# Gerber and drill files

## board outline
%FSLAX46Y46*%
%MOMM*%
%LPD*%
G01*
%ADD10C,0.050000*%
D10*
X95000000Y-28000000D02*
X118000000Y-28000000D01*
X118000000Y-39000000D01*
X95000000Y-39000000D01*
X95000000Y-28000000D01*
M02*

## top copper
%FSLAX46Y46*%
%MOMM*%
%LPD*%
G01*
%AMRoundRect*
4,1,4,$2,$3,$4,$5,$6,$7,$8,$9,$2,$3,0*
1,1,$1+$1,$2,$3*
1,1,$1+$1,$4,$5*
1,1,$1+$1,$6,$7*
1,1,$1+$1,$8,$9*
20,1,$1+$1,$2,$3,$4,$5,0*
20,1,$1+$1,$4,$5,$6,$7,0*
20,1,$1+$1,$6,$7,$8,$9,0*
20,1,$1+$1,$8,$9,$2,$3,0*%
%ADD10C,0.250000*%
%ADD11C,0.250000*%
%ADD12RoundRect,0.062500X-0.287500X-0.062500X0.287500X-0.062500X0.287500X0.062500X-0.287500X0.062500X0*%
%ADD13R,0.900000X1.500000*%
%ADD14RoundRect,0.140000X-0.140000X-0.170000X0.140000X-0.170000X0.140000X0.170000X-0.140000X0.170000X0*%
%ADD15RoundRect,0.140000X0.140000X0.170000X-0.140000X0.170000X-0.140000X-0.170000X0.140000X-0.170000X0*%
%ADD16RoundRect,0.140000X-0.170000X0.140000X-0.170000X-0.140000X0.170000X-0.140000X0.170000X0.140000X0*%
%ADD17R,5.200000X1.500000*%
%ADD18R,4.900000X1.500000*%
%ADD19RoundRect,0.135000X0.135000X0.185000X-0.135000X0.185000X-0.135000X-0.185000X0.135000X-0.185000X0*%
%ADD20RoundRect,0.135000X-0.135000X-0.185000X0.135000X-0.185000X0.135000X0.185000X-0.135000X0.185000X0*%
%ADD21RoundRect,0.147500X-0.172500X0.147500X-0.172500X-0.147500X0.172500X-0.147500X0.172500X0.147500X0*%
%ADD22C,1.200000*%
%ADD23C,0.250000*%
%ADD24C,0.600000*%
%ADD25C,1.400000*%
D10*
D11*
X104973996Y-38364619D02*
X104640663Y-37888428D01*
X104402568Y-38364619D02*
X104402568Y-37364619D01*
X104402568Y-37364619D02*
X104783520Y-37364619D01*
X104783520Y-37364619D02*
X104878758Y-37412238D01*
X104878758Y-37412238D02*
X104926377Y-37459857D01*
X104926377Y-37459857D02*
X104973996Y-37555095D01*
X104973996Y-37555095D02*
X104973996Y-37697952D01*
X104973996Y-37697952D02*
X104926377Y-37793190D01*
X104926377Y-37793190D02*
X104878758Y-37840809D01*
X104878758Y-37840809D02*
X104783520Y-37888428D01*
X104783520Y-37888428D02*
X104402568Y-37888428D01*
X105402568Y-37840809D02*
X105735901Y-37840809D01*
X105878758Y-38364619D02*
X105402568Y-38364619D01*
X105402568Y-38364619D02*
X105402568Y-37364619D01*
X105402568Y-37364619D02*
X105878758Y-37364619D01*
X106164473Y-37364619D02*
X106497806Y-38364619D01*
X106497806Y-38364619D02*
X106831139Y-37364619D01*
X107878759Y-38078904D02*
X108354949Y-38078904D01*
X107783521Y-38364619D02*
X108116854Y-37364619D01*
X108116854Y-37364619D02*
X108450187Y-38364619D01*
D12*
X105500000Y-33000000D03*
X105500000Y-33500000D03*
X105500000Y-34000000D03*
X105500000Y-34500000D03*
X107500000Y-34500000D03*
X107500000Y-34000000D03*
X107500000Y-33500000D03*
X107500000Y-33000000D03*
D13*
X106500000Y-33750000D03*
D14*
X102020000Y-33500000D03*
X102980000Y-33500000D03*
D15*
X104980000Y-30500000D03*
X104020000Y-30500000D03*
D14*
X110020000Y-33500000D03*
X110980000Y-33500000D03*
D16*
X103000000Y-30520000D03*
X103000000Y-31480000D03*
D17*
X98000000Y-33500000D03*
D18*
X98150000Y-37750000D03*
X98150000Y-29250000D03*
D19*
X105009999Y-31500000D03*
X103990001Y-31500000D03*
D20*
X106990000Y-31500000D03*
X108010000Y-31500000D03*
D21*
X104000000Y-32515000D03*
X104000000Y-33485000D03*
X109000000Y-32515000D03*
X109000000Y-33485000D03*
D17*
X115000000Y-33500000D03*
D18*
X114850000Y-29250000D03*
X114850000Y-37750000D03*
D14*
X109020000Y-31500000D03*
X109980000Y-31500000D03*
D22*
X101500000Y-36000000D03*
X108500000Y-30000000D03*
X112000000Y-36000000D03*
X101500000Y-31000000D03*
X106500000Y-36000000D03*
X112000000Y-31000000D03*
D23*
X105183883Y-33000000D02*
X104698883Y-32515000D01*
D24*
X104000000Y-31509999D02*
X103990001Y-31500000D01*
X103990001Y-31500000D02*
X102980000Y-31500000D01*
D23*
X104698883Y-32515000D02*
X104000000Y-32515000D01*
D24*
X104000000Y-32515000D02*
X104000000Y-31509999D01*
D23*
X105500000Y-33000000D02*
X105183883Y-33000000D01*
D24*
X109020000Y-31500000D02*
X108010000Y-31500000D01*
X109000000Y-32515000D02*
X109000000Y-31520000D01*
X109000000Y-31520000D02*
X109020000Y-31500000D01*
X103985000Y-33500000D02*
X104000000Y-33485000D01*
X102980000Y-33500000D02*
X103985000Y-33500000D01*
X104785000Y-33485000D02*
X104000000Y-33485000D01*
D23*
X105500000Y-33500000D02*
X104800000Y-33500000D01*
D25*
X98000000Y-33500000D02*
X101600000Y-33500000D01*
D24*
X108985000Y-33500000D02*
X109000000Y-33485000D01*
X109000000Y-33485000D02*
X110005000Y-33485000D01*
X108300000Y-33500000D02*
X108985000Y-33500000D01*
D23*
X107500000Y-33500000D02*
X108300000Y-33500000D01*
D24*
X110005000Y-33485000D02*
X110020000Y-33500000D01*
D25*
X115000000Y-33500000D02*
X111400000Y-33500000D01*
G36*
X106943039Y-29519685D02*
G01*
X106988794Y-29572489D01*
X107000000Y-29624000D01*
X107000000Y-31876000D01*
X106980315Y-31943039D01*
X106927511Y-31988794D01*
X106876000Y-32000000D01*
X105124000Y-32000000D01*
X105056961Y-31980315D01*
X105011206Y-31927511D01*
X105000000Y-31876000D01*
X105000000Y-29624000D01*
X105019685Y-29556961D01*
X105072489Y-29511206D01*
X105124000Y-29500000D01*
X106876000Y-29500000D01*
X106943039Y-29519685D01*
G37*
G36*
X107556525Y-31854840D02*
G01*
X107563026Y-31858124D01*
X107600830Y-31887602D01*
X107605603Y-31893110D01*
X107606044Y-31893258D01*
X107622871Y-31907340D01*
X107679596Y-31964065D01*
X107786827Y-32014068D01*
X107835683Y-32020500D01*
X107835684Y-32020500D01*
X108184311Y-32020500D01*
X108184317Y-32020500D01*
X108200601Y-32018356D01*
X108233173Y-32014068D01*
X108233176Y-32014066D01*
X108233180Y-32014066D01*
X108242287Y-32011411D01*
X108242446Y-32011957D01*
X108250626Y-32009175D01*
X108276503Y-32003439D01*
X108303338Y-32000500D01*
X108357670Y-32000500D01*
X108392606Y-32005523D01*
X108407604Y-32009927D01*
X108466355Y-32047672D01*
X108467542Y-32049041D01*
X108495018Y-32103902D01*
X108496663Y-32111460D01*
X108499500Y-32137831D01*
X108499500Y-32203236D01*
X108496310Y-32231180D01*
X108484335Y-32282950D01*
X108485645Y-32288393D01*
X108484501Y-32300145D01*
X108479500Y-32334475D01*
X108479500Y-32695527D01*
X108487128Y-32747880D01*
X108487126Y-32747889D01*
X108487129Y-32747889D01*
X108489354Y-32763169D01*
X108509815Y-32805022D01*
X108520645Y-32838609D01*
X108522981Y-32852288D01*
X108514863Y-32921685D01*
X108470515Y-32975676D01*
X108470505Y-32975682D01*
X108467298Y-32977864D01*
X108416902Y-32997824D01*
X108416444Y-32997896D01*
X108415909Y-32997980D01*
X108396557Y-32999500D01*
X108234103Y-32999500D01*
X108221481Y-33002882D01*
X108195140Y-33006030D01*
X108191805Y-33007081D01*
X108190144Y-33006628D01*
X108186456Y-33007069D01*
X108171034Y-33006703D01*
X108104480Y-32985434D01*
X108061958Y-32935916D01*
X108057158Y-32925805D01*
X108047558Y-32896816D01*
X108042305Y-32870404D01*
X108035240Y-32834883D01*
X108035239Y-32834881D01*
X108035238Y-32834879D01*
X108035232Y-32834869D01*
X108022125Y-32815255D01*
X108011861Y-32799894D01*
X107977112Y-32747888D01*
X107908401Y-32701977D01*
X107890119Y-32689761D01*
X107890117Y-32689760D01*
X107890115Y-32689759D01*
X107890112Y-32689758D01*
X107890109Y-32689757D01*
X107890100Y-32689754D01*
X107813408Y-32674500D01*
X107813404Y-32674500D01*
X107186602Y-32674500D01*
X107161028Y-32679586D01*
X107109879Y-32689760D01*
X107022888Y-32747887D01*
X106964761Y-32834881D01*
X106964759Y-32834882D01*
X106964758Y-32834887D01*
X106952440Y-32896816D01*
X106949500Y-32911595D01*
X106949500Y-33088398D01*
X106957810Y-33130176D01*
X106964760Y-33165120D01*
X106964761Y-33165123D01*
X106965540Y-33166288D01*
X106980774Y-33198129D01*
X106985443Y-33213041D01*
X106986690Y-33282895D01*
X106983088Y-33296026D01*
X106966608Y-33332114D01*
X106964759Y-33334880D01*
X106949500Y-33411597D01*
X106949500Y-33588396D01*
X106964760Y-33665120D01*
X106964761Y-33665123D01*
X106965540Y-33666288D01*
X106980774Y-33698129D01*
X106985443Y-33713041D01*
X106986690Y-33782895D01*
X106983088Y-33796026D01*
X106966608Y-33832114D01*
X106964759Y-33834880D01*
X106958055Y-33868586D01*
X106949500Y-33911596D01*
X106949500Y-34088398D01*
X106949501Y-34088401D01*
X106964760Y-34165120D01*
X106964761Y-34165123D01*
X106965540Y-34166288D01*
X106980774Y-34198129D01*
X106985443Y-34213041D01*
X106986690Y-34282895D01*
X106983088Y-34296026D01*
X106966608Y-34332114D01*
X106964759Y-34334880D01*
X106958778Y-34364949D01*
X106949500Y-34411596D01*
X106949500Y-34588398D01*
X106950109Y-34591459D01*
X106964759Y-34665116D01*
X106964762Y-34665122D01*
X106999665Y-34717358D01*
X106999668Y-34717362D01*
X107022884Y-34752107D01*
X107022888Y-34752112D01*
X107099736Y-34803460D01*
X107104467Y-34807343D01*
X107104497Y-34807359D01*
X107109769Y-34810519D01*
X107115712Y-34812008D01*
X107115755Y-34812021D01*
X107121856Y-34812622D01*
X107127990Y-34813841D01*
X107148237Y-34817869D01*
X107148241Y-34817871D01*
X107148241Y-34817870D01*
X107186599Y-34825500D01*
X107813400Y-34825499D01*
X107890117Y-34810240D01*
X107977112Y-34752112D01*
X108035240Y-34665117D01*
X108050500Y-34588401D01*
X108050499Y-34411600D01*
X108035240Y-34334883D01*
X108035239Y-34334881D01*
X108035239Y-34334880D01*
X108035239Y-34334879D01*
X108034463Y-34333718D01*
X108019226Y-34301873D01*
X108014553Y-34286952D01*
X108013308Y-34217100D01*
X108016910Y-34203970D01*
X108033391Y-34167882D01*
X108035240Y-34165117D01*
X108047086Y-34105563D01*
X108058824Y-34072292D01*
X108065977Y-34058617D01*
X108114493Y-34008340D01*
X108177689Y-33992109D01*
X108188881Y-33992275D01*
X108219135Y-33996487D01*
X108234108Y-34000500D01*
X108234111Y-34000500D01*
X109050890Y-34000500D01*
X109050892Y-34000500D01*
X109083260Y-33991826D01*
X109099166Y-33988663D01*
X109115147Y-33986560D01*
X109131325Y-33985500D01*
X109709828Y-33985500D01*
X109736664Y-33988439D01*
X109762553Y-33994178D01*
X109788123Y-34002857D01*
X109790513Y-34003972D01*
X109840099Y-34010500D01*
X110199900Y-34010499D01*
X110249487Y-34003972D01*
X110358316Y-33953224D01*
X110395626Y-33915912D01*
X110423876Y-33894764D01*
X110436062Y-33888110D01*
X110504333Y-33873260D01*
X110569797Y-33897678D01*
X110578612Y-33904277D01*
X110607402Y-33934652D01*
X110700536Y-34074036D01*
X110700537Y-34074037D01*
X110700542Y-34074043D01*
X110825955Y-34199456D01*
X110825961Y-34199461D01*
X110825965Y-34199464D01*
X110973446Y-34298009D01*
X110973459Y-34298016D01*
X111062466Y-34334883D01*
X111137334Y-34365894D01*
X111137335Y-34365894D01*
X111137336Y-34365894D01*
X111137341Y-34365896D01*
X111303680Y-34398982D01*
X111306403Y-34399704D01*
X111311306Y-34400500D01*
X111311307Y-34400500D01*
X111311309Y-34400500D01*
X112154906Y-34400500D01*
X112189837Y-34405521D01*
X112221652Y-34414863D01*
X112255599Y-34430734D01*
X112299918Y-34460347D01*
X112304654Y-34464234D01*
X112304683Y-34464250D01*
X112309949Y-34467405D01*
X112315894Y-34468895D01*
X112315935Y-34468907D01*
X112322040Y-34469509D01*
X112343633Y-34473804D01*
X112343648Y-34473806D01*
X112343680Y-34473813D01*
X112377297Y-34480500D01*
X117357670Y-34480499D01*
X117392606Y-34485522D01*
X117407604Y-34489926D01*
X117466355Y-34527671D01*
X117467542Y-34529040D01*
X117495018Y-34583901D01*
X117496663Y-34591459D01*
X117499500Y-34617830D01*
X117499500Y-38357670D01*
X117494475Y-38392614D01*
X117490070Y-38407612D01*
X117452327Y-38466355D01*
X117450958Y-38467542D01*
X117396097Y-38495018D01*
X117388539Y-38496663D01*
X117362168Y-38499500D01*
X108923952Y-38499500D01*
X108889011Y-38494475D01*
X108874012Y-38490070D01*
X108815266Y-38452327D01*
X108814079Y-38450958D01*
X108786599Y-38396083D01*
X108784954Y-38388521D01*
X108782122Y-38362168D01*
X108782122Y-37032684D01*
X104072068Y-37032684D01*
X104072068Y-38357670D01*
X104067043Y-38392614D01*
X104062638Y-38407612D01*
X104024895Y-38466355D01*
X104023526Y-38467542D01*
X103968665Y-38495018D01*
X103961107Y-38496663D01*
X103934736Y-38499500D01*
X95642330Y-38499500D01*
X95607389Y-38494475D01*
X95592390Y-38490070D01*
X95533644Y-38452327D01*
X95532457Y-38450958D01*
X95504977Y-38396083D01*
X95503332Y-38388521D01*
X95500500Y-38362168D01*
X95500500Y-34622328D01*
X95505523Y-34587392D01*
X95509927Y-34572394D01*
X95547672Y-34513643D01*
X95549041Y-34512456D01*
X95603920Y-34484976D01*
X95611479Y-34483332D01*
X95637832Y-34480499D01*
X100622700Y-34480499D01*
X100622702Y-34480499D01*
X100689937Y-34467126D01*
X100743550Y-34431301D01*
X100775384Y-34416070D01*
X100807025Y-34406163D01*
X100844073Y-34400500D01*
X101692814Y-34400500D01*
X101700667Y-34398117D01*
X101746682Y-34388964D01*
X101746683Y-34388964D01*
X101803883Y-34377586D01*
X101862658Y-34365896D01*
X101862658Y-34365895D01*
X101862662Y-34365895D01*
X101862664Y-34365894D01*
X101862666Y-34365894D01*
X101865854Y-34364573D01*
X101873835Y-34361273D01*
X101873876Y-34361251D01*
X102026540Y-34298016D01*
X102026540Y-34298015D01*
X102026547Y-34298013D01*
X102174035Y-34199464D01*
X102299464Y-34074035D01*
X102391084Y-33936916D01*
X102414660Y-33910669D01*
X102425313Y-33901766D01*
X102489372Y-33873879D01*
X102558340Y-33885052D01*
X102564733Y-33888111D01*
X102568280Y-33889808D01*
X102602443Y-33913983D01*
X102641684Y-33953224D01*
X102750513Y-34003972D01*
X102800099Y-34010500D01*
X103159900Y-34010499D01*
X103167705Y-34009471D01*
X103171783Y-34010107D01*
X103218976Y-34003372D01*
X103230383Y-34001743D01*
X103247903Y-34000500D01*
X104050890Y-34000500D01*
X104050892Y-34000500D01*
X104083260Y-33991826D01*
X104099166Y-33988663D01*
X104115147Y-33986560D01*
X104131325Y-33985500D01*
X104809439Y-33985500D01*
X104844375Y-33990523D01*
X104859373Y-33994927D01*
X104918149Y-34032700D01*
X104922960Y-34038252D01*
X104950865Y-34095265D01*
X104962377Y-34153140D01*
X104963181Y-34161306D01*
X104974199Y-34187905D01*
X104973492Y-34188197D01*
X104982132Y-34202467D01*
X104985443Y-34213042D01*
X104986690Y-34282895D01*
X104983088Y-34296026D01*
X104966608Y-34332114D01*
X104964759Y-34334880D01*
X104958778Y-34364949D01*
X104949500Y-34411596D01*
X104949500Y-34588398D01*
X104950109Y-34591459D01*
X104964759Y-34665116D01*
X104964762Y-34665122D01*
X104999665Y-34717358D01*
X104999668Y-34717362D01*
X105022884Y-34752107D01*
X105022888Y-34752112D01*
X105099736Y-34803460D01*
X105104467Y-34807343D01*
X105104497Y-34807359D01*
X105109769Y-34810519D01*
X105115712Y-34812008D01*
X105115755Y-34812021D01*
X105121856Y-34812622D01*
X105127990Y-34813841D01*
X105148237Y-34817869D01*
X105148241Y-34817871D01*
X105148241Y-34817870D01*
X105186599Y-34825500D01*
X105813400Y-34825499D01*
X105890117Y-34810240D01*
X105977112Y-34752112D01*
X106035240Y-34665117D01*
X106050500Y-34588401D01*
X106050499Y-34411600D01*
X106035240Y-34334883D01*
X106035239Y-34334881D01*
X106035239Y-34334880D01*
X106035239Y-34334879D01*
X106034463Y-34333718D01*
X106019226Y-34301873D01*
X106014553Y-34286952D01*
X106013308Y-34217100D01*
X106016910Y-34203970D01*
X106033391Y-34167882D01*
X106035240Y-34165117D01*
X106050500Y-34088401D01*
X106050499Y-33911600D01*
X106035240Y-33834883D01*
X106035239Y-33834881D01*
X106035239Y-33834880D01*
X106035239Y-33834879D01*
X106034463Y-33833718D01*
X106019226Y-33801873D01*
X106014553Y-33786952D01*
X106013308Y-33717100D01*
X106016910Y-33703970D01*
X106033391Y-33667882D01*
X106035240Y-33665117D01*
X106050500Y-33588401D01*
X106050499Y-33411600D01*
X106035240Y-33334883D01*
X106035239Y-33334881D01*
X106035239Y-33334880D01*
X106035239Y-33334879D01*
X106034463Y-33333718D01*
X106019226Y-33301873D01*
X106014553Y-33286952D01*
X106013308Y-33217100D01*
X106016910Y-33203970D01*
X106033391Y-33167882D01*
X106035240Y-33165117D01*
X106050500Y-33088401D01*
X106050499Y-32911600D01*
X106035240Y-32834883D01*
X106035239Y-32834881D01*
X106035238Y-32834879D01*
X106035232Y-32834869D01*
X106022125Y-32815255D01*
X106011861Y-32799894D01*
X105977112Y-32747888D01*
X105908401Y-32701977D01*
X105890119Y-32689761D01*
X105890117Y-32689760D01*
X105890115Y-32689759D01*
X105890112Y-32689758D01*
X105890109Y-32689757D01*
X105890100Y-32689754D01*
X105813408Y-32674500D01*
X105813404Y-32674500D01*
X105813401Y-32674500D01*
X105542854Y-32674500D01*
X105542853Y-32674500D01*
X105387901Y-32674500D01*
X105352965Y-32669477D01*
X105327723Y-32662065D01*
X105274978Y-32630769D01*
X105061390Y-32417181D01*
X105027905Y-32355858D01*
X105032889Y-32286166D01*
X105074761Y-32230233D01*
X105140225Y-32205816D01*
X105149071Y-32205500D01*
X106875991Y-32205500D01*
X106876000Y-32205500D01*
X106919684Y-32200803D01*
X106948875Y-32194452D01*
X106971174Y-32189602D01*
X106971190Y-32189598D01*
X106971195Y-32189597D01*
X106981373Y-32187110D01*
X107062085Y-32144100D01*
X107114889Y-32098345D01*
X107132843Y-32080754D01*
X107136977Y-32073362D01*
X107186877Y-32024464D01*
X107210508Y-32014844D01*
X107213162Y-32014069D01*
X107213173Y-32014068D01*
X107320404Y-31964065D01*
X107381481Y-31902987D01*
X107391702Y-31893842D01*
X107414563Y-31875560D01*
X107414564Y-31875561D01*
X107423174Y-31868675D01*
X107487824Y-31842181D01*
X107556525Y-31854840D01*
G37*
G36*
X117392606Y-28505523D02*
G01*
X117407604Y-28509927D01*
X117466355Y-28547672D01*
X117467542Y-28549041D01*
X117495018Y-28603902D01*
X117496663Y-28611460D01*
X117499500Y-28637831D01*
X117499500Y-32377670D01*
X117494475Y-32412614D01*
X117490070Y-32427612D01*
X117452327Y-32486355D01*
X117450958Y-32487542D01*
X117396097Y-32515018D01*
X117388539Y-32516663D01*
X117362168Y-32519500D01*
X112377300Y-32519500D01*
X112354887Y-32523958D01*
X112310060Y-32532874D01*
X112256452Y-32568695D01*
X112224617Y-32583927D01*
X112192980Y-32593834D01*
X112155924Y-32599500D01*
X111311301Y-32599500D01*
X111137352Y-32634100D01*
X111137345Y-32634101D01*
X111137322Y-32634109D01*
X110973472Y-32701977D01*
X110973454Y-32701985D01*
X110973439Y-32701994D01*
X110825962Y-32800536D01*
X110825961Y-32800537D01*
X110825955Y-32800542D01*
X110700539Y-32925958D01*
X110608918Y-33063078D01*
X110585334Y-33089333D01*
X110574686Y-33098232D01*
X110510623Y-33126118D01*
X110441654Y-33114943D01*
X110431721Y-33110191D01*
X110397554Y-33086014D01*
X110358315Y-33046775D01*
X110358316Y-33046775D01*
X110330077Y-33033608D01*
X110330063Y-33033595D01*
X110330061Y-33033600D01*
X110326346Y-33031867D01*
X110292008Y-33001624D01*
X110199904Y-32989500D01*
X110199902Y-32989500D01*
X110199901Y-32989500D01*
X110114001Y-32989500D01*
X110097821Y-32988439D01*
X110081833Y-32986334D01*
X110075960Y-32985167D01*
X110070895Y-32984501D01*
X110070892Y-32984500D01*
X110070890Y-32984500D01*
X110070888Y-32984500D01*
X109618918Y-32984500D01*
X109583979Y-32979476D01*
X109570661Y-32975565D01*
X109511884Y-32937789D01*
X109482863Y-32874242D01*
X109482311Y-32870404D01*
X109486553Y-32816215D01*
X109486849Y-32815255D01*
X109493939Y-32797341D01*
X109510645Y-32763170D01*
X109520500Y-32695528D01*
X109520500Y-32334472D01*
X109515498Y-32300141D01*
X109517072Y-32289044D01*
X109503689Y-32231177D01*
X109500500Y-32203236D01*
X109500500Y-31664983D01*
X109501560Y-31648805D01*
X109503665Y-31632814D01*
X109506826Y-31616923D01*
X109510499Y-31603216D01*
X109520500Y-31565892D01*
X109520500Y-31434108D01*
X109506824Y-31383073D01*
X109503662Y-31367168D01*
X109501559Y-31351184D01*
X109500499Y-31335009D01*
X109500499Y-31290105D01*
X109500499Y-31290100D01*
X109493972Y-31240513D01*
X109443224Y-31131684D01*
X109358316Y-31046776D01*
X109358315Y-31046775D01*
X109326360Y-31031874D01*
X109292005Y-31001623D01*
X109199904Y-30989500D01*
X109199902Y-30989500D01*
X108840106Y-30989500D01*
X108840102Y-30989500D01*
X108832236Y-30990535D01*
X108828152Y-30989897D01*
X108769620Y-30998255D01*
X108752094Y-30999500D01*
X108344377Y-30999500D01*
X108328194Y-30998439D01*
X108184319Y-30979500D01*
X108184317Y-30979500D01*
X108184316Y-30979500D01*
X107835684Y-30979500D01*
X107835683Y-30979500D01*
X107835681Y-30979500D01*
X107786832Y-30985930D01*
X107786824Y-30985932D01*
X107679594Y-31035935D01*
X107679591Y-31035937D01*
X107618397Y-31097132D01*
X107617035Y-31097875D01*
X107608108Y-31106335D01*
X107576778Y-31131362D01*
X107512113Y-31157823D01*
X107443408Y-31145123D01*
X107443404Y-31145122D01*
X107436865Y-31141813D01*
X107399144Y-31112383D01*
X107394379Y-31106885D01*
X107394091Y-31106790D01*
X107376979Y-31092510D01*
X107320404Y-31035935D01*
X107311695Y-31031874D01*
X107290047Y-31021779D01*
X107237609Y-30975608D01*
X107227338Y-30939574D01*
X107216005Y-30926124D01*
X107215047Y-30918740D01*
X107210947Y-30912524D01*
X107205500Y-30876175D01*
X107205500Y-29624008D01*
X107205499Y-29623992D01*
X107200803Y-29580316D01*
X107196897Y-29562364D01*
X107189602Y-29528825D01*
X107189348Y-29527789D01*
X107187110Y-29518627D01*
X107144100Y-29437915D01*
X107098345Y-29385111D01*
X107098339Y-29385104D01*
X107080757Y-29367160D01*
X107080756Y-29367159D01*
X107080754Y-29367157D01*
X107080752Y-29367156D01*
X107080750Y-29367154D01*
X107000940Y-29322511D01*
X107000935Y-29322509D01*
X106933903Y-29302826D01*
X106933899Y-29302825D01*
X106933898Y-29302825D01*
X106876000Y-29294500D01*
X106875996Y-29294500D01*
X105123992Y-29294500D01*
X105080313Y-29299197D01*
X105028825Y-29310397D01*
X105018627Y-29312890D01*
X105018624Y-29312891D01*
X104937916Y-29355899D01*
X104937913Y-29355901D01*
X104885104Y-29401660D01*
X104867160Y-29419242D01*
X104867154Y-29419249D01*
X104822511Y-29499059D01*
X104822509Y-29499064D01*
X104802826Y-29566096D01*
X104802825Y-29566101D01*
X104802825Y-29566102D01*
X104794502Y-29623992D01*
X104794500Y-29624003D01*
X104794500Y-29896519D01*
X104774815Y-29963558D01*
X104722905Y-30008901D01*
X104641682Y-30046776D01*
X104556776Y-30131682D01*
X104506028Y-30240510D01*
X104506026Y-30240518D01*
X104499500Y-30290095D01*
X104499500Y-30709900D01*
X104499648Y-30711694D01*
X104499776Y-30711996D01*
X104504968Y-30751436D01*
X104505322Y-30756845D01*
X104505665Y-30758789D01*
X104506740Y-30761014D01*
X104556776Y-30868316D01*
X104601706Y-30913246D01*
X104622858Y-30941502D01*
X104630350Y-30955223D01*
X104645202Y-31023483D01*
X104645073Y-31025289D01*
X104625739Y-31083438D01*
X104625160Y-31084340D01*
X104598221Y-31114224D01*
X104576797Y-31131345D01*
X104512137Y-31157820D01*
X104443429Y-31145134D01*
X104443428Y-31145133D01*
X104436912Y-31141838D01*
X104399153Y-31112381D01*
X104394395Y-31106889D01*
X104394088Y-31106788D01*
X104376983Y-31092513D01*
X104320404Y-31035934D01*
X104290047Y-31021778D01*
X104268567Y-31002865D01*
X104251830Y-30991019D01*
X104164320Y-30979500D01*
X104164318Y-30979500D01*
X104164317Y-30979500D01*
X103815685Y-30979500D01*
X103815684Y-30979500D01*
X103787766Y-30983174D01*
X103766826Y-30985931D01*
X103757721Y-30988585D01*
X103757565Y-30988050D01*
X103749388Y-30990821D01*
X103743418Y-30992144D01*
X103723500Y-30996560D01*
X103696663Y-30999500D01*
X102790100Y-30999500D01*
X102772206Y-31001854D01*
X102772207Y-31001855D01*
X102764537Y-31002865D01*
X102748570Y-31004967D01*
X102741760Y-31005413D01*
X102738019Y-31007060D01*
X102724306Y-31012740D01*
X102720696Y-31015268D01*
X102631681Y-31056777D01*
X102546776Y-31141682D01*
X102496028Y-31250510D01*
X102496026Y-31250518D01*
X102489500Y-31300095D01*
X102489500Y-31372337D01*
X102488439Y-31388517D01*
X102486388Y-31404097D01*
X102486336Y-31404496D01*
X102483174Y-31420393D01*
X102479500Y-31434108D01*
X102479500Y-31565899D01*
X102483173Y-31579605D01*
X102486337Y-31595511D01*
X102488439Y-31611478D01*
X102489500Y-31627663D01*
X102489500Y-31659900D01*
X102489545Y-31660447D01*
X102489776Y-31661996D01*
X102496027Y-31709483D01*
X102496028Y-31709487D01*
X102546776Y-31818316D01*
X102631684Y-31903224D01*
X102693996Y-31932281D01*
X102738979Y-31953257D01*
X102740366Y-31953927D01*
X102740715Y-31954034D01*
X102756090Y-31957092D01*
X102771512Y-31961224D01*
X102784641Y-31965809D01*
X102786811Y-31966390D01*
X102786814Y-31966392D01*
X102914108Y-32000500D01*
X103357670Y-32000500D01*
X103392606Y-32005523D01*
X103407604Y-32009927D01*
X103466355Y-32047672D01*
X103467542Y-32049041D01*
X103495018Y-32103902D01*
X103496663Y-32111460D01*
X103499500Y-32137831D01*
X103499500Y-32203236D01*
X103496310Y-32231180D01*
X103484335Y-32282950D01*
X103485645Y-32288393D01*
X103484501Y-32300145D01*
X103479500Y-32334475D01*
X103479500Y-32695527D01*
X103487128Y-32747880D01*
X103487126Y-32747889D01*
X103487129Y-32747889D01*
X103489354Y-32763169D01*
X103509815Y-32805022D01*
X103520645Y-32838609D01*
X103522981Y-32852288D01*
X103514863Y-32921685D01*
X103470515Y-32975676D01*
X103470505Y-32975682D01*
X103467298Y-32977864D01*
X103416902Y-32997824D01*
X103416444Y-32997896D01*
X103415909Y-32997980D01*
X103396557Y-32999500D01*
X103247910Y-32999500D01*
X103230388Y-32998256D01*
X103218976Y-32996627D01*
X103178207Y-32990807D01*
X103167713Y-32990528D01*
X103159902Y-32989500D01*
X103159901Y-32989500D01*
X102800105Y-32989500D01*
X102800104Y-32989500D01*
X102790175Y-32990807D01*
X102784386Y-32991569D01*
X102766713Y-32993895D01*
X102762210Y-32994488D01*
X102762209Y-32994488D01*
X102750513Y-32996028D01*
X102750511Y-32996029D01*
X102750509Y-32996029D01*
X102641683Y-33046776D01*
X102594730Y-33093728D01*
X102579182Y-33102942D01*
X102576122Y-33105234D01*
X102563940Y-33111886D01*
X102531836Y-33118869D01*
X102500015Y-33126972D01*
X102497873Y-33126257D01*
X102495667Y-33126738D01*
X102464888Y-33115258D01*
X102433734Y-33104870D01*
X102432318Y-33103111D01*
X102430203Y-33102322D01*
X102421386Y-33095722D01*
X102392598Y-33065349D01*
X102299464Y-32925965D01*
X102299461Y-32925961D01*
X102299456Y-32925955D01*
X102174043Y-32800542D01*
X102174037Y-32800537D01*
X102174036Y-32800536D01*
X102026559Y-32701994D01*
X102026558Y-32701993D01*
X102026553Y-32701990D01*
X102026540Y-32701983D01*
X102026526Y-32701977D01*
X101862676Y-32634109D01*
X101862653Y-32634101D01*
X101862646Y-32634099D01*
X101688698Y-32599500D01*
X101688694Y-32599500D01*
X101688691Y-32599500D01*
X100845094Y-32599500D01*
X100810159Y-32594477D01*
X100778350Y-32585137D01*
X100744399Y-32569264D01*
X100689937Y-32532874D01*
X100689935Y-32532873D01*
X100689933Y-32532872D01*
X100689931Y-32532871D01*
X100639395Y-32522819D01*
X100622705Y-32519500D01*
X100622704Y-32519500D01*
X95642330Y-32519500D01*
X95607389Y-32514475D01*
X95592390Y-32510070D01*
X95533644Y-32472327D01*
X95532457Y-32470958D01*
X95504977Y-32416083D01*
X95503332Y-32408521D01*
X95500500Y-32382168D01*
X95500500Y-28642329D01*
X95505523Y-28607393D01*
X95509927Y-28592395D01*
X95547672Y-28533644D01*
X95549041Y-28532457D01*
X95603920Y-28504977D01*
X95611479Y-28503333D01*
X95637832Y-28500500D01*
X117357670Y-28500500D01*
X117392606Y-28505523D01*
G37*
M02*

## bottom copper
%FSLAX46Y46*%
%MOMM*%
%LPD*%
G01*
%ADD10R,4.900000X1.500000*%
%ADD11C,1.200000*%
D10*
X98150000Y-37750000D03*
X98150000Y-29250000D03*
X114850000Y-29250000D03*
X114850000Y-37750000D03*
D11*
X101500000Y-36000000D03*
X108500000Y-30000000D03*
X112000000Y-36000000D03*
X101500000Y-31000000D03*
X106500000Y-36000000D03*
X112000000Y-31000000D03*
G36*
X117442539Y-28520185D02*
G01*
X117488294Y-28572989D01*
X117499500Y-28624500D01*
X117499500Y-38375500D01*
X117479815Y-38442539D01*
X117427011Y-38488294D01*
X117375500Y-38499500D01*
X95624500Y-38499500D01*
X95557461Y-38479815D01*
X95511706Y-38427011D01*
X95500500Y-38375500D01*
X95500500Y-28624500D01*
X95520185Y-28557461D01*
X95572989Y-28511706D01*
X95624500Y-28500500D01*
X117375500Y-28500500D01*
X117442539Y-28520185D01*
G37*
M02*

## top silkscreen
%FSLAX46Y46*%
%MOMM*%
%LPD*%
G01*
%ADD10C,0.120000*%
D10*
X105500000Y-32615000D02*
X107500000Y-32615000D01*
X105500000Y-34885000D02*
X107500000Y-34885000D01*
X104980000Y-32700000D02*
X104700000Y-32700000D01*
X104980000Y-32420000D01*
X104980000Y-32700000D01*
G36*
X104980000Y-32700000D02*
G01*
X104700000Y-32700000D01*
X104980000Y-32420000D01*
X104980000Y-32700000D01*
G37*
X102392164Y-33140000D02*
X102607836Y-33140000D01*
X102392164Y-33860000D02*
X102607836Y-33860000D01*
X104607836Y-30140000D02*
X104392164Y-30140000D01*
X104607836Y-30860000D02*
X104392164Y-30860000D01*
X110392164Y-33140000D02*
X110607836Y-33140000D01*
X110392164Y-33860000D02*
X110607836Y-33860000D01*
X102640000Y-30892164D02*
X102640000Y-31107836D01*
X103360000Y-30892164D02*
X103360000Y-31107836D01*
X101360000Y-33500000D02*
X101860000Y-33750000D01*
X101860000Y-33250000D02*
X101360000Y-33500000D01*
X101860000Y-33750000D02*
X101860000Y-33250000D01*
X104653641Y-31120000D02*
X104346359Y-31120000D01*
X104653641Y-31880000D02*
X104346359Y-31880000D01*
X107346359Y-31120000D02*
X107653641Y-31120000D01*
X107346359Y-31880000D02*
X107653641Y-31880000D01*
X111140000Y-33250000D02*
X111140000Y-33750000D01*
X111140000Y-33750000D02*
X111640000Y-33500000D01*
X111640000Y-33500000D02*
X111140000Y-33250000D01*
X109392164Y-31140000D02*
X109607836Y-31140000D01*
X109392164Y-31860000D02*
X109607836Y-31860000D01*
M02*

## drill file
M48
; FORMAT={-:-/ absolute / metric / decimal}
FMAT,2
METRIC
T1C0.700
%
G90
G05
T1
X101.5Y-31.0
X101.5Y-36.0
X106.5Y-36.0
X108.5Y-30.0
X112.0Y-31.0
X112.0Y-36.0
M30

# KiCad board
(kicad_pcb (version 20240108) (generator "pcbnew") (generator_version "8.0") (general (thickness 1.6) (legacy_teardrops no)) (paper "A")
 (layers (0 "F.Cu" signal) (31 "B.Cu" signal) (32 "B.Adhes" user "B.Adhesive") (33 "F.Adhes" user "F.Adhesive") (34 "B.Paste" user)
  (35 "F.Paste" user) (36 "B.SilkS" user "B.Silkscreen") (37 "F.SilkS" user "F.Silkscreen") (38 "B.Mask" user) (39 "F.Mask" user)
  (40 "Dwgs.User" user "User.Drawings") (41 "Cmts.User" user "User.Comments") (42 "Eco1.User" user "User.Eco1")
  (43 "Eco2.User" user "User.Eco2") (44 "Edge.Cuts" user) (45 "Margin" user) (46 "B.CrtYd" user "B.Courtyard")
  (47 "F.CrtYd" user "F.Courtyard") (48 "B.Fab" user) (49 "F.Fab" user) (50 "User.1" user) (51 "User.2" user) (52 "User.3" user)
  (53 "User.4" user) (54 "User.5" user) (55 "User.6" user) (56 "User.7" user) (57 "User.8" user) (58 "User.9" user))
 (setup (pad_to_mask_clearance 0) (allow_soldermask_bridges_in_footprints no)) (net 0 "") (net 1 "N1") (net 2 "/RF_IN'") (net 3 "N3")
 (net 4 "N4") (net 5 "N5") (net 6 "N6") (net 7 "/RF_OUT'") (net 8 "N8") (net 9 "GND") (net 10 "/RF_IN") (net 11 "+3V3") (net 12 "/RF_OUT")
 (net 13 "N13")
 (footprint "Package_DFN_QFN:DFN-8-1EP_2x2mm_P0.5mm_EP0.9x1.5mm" (layer "F.Cu") (at 106.5 33.75)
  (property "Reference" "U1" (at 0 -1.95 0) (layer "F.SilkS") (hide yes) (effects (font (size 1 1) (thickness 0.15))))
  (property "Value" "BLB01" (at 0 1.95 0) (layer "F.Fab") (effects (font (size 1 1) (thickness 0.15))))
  (fp_line (start -1 -1.135) (end 1 -1.135) (stroke (width 0.12) (type solid)) (layer "F.SilkS"))
  (fp_line (start -1 1.135) (end 1 1.135) (stroke (width 0.12) (type solid)) (layer "F.SilkS"))
  (fp_poly
   (pts (xy -1.52 -1.05) (xy -1.8 -1.05) (xy -1.52 -1.33) (xy -1.52 -1.05)) (stroke (width 0.12) (type solid)) (fill solid)
   (layer "F.SilkS"))
  (pad "" smd roundrect (at -0.225 -0.375) (size 0.36 0.6) (layers "F.Paste") (roundrect_rratio 0.25))
  (pad "" smd roundrect (at -0.225 0.375) (size 0.36 0.6) (layers "F.Paste") (roundrect_rratio 0.25))
  (pad "" smd roundrect (at 0.225 -0.375) (size 0.36 0.6) (layers "F.Paste") (roundrect_rratio 0.25))
  (pad "" smd roundrect (at 0.225 0.375) (size 0.36 0.6) (layers "F.Paste") (roundrect_rratio 0.25))
  (pad "1" smd roundrect (at -1 -0.75) (size 0.7 0.25) (layers "F.Cu" "F.Paste" "F.Mask") (roundrect_rratio 0.25) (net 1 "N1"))
  (pad "2" smd roundrect (at -1 -0.25) (size 0.7 0.25) (layers "F.Cu" "F.Paste" "F.Mask") (roundrect_rratio 0.25) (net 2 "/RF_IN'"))
  (pad "3" smd roundrect (at -1 0.25) (size 0.7 0.25) (layers "F.Cu" "F.Paste" "F.Mask") (roundrect_rratio 0.25) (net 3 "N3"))
  (pad "4" smd roundrect (at -1 0.75) (size 0.7 0.25) (layers "F.Cu" "F.Paste" "F.Mask") (roundrect_rratio 0.25) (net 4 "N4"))
  (pad "5" smd roundrect (at 1 0.75) (size 0.7 0.25) (layers "F.Cu" "F.Paste" "F.Mask") (roundrect_rratio 0.25) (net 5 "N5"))
  (pad "6" smd roundrect (at 1 0.25) (size 0.7 0.25) (layers "F.Cu" "F.Paste" "F.Mask") (roundrect_rratio 0.25) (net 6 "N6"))
  (pad "7" smd roundrect (at 1 -0.25) (size 0.7 0.25) (layers "F.Cu" "F.Paste" "F.Mask") (roundrect_rratio 0.25) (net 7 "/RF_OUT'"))
  (pad "8" smd roundrect (at 1 -0.75) (size 0.7 0.25) (layers "F.Cu" "F.Paste" "F.Mask") (roundrect_rratio 0.25) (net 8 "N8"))
  (pad "9" smd rect (at 0 0) (size 0.9 1.5) (layers "F.Cu" "F.Mask") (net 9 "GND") (zone_connect 2)))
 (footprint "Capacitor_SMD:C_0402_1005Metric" (layer "F.Cu") (at 102.5 33.5)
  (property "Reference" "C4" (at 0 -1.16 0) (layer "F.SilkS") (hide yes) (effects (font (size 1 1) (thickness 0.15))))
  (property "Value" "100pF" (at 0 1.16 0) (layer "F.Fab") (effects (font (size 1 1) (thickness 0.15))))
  (fp_line (start -0.107836 -0.36) (end 0.107836 -0.36) (stroke (width 0.12) (type solid)) (layer "F.SilkS"))
  (fp_line (start -0.107836 0.36) (end 0.107836 0.36) (stroke (width 0.12) (type solid)) (layer "F.SilkS"))
  (pad "1" smd roundrect (at -0.48 0) (size 0.56 0.62) (layers "F.Cu" "F.Paste" "F.Mask") (roundrect_rratio 0.25) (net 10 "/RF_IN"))
  (pad "2" smd roundrect (at 0.48 0) (size 0.56 0.62) (layers "F.Cu" "F.Paste" "F.Mask") (roundrect_rratio 0.25) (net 2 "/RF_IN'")))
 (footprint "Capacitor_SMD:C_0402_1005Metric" (layer "F.Cu") (at 104.5 30.5 180)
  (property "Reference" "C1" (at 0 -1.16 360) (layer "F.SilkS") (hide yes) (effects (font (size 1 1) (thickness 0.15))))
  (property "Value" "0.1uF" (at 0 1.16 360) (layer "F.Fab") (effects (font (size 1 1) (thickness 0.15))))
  (fp_line (start -0.107836 0.36) (end 0.107836 0.36) (stroke (width 0.12) (type solid)) (layer "F.SilkS"))
  (fp_line (start -0.107836 -0.36) (end 0.107836 -0.36) (stroke (width 0.12) (type solid)) (layer "F.SilkS"))
  (pad "1" smd roundrect (at -0.48 0 180) (size 0.56 0.62) (layers "F.Cu" "F.Paste" "F.Mask") (roundrect_rratio 0.25) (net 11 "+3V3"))
  (pad "2" smd roundrect (at 0.48 0 180) (size 0.56 0.62) (layers "F.Cu" "F.Paste" "F.Mask") (roundrect_rratio 0.25) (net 9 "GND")))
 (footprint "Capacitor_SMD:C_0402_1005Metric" (layer "F.Cu") (at 110.5 33.5)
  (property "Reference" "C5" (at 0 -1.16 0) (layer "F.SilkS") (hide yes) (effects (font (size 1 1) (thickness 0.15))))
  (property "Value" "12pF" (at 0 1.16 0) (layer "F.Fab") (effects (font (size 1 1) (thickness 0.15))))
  (fp_line (start -0.107836 -0.36) (end 0.107836 -0.36) (stroke (width 0.12) (type solid)) (layer "F.SilkS"))
  (fp_line (start -0.107836 0.36) (end 0.107836 0.36) (stroke (width 0.12) (type solid)) (layer "F.SilkS"))
  (pad "1" smd roundrect (at -0.48 0) (size 0.56 0.62) (layers "F.Cu" "F.Paste" "F.Mask") (roundrect_rratio 0.25) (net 7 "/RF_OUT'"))
  (pad "2" smd roundrect (at 0.48 0) (size 0.56 0.62) (layers "F.Cu" "F.Paste" "F.Mask") (roundrect_rratio 0.25) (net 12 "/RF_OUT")))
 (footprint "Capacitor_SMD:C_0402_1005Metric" (layer "F.Cu") (at 103 31 -90)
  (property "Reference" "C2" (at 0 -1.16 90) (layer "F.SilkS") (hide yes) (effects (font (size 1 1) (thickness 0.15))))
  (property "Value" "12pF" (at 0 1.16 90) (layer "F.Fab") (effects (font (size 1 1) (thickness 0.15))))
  (fp_line (start -0.107836 0.36) (end 0.107836 0.36) (stroke (width 0.12) (type solid)) (layer "F.SilkS"))
  (fp_line (start -0.107836 -0.36) (end 0.107836 -0.36) (stroke (width 0.12) (type solid)) (layer "F.SilkS"))
  (pad "1" smd roundrect (at -0.48 0 270) (size 0.56 0.62) (layers "F.Cu" "F.Paste" "F.Mask") (roundrect_rratio 0.25) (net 9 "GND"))
  (pad "2" smd roundrect (at 0.48 0 270) (size 0.56 0.62) (layers "F.Cu" "F.Paste" "F.Mask") (roundrect_rratio 0.25) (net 1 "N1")))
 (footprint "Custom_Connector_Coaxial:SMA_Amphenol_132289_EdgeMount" (layer "F.Cu") (at 98.15 33.5 180)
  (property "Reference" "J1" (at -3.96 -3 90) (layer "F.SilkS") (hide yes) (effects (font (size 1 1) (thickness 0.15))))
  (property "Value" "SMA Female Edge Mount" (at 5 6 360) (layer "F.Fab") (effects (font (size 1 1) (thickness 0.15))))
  (fp_line (start -3.21 0) (end -3.71 -0.25) (stroke (width 0.12) (type solid)) (layer "F.SilkS"))
  (fp_line (start -3.71 0.25) (end -3.21 0) (stroke (width 0.12) (type solid)) (layer "F.SilkS"))
  (fp_line (start -3.71 -0.25) (end -3.71 0.25) (stroke (width 0.12) (type solid)) (layer "F.SilkS"))
  (pad "1" smd rect (at 0.15 0 270) (size 1.5 5.2) (layers "F.Cu" "F.Paste" "F.Mask") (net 10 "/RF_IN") (clearance 0.23))
  (pad "2" smd rect (at 0 -4.25 270) (size 1.5 4.9) (layers "F.Cu" "F.Paste" "F.Mask") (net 9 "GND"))
  (pad "2" smd rect (at 0 -4.25 270) (size 1.5 4.9) (layers "B.Cu" "B.Paste" "B.Mask") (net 9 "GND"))
  (pad "2" smd rect (at 0 4.25 270) (size 1.5 4.9) (layers "F.Cu" "F.Paste" "F.Mask") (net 9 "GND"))
  (pad "2" smd rect (at 0 4.25 270) (size 1.5 4.9) (layers "B.Cu" "B.Paste" "B.Mask") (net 9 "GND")))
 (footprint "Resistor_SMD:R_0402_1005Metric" (layer "F.Cu") (at 104.5 31.5 180)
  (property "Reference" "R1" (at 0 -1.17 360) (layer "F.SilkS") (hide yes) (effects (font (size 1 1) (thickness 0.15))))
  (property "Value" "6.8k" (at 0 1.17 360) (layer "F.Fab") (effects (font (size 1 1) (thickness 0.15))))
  (fp_line (start -0.153641 0.38) (end 0.153641 0.38) (stroke (width 0.12) (type solid)) (layer "F.SilkS"))
  (fp_line (start -0.153641 -0.38) (end 0.153641 -0.38) (stroke (width 0.12) (type solid)) (layer "F.SilkS"))
  (pad "1" smd roundrect (at -0.509999 0 180) (size 0.54 0.64) (layers "F.Cu" "F.Paste" "F.Mask") (roundrect_rratio 0.25) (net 11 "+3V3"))
  (pad "2" smd roundrect (at 0.509999 0 180) (size 0.54 0.64) (layers "F.Cu" "F.Paste" "F.Mask") (roundrect_rratio 0.25) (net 1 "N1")))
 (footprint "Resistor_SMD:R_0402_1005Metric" (layer "F.Cu") (at 107.5 31.5)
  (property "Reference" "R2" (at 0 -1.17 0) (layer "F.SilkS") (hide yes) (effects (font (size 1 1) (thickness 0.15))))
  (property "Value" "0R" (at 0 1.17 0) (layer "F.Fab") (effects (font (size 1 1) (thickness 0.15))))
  (fp_line (start -0.153641 -0.38) (end 0.153641 -0.38) (stroke (width 0.12) (type solid)) (layer "F.SilkS"))
  (fp_line (start -0.153641 0.38) (end 0.153641 0.38) (stroke (width 0.12) (type solid)) (layer "F.SilkS"))
  (pad "1" smd roundrect (at -0.51 0) (size 0.54 0.64) (layers "F.Cu" "F.Paste" "F.Mask") (roundrect_rratio 0.25) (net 11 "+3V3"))
  (pad "2" smd roundrect (at 0.51 0) (size 0.54 0.64) (layers "F.Cu" "F.Paste" "F.Mask") (roundrect_rratio 0.25) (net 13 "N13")))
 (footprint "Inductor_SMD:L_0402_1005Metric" (layer "F.Cu") (at 104 33 -90)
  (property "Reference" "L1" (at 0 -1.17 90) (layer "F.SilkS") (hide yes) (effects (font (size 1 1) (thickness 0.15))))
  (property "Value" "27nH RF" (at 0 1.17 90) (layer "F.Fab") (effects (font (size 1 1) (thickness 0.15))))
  (pad "1" smd roundrect (at -0.485 0 270) (size 0.59 0.64) (layers "F.Cu" "F.Paste" "F.Mask") (roundrect_rratio 0.25) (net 1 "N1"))
  (pad "2" smd roundrect (at 0.485 0 270) (size 0.59 0.64) (layers "F.Cu" "F.Paste" "F.Mask") (roundrect_rratio 0.25) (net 2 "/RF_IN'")))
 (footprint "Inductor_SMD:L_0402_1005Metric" (layer "F.Cu") (at 109 33 -90)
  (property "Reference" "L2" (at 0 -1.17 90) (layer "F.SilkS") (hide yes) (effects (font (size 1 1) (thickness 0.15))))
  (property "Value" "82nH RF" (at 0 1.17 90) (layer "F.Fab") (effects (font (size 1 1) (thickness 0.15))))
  (pad "1" smd roundrect (at -0.485 0 270) (size 0.59 0.64) (layers "F.Cu" "F.Paste" "F.Mask") (roundrect_rratio 0.25) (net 13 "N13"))
  (pad "2" smd roundrect (at 0.485 0 270) (size 0.59 0.64) (layers "F.Cu" "F.Paste" "F.Mask") (roundrect_rratio 0.25) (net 7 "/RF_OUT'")))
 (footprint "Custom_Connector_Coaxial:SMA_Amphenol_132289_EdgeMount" (layer "F.Cu") (at 114.85 33.5)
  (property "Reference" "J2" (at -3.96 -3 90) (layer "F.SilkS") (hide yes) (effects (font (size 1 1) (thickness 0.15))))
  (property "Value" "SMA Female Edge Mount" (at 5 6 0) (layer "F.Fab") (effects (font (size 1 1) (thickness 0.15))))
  (fp_line (start -3.71 -0.25) (end -3.71 0.25) (stroke (width 0.12) (type solid)) (layer "F.SilkS"))
  (fp_line (start -3.71 0.25) (end -3.21 0) (stroke (width 0.12) (type solid)) (layer "F.SilkS"))
  (fp_line (start -3.21 0) (end -3.71 -0.25) (stroke (width 0.12) (type solid)) (layer "F.SilkS"))
  (pad "1" smd rect (at 0.15 0 90) (size 1.5 5.2) (layers "F.Cu" "F.Paste" "F.Mask") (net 12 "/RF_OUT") (clearance 0.23))
  (pad "2" smd rect (at 0 -4.25 90) (size 1.5 4.9) (layers "F.Cu" "F.Paste" "F.Mask") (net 9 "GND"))
  (pad "2" smd rect (at 0 -4.25 90) (size 1.5 4.9) (layers "B.Cu" "B.Paste" "B.Mask") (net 9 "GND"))
  (pad "2" smd rect (at 0 4.25 90) (size 1.5 4.9) (layers "F.Cu" "F.Paste" "F.Mask") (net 9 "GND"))
  (pad "2" smd rect (at 0 4.25 90) (size 1.5 4.9) (layers "B.Cu" "B.Paste" "B.Mask") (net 9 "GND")))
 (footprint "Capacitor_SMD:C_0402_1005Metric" (layer "F.Cu") (at 109.5 31.5)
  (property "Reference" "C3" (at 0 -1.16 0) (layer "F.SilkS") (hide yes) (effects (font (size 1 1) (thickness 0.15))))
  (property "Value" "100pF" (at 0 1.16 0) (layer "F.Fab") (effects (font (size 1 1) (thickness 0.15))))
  (fp_line (start -0.107836 -0.36) (end 0.107836 -0.36) (stroke (width 0.12) (type solid)) (layer "F.SilkS"))
  (fp_line (start -0.107836 0.36) (end 0.107836 0.36) (stroke (width 0.12) (type solid)) (layer "F.SilkS"))
  (pad "1" smd roundrect (at -0.48 0) (size 0.56 0.62) (layers "F.Cu" "F.Paste" "F.Mask") (roundrect_rratio 0.25) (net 13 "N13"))
  (pad "2" smd roundrect (at 0.48 0) (size 0.56 0.62) (layers "F.Cu" "F.Paste" "F.Mask") (roundrect_rratio 0.25) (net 9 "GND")))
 (gr_rect (start 95 28) (end 118 39) (stroke (width 0.05) (type default)) (fill none) (layer "Edge.Cuts"))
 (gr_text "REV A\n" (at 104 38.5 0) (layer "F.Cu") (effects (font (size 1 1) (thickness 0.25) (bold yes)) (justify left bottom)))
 (via (at 101.5 36) (size 1.2) (drill 0.7) (layers "F.Cu" "B.Cu") (free yes) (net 9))
 (via (at 108.5 30) (size 1.2) (drill 0.7) (layers "F.Cu" "B.Cu") (free yes) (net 9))
 (via (at 112 36) (size 1.2) (drill 0.7) (layers "F.Cu" "B.Cu") (free yes) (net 9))
 (via (at 101.5 31) (size 1.2) (drill 0.7) (layers "F.Cu" "B.Cu") (free yes) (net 9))
 (via (at 106.5 36) (size 1.2) (drill 0.7) (layers "F.Cu" "B.Cu") (free yes) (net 9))
 (via (at 112 31) (size 1.2) (drill 0.7) (layers "F.Cu" "B.Cu") (free yes) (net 9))
 (segment (start 105.183883 33) (end 104.698883 32.515) (width 0.25) (layer "F.Cu") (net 1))
 (segment (start 104 31.509999) (end 103.990001 31.5) (width 0.6) (layer "F.Cu") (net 1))
 (segment (start 103.990001 31.5) (end 102.98 31.5) (width 0.6) (layer "F.Cu") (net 1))
 (segment (start 104.698883 32.515) (end 104 32.515) (width 0.25) (layer "F.Cu") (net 1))
 (segment (start 104 32.515) (end 104 31.509999) (width 0.6) (layer "F.Cu") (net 1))
 (segment (start 105.5 33) (end 105.183883 33) (width 0.25) (layer "F.Cu") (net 1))
 (segment (start 109.02 31.5) (end 108.01 31.5) (width 0.6) (layer "F.Cu") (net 13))
 (segment (start 109 32.515) (end 109 31.52) (width 0.6) (layer "F.Cu") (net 13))
 (segment (start 109 31.52) (end 109.02 31.5) (width 0.6) (layer "F.Cu") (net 13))
 (segment (start 103.985 33.5) (end 104 33.485) (width 0.6) (layer "F.Cu") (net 2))
 (segment (start 102.98 33.5) (end 103.985 33.5) (width 0.6) (layer "F.Cu") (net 2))
 (segment (start 104.785 33.485) (end 104 33.485) (width 0.6) (layer "F.Cu") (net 2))
 (segment (start 105.5 33.5) (end 104.8 33.5) (width 0.25) (layer "F.Cu") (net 2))
 (segment (start 98 33.5) (end 101.6 33.5) (width 1.4) (layer "F.Cu") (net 10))
 (segment (start 108.985 33.5) (end 109 33.485) (width 0.6) (layer "F.Cu") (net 7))
 (segment (start 109 33.485) (end 110.005 33.485) (width 0.6) (layer "F.Cu") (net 7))
 (segment (start 108.3 33.5) (end 108.985 33.5) (width 0.6) (layer "F.Cu") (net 7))
 (segment (start 107.5 33.5) (end 108.3 33.5) (width 0.25) (layer "F.Cu") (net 7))
 (segment (start 110.005 33.485) (end 110.02 33.5) (width 0.6) (layer "F.Cu") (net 7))
 (segment (start 115 33.5) (end 111.4 33.5) (width 1.4) (layer "F.Cu") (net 12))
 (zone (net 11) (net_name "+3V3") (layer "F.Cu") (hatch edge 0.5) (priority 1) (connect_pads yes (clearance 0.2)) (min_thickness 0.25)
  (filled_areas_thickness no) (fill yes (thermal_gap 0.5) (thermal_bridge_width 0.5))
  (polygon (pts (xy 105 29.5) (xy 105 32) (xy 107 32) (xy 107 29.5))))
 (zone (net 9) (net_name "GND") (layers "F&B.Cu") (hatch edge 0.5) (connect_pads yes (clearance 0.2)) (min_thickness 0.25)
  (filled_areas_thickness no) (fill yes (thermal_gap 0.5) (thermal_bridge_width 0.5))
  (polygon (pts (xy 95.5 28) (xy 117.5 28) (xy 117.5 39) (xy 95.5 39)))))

